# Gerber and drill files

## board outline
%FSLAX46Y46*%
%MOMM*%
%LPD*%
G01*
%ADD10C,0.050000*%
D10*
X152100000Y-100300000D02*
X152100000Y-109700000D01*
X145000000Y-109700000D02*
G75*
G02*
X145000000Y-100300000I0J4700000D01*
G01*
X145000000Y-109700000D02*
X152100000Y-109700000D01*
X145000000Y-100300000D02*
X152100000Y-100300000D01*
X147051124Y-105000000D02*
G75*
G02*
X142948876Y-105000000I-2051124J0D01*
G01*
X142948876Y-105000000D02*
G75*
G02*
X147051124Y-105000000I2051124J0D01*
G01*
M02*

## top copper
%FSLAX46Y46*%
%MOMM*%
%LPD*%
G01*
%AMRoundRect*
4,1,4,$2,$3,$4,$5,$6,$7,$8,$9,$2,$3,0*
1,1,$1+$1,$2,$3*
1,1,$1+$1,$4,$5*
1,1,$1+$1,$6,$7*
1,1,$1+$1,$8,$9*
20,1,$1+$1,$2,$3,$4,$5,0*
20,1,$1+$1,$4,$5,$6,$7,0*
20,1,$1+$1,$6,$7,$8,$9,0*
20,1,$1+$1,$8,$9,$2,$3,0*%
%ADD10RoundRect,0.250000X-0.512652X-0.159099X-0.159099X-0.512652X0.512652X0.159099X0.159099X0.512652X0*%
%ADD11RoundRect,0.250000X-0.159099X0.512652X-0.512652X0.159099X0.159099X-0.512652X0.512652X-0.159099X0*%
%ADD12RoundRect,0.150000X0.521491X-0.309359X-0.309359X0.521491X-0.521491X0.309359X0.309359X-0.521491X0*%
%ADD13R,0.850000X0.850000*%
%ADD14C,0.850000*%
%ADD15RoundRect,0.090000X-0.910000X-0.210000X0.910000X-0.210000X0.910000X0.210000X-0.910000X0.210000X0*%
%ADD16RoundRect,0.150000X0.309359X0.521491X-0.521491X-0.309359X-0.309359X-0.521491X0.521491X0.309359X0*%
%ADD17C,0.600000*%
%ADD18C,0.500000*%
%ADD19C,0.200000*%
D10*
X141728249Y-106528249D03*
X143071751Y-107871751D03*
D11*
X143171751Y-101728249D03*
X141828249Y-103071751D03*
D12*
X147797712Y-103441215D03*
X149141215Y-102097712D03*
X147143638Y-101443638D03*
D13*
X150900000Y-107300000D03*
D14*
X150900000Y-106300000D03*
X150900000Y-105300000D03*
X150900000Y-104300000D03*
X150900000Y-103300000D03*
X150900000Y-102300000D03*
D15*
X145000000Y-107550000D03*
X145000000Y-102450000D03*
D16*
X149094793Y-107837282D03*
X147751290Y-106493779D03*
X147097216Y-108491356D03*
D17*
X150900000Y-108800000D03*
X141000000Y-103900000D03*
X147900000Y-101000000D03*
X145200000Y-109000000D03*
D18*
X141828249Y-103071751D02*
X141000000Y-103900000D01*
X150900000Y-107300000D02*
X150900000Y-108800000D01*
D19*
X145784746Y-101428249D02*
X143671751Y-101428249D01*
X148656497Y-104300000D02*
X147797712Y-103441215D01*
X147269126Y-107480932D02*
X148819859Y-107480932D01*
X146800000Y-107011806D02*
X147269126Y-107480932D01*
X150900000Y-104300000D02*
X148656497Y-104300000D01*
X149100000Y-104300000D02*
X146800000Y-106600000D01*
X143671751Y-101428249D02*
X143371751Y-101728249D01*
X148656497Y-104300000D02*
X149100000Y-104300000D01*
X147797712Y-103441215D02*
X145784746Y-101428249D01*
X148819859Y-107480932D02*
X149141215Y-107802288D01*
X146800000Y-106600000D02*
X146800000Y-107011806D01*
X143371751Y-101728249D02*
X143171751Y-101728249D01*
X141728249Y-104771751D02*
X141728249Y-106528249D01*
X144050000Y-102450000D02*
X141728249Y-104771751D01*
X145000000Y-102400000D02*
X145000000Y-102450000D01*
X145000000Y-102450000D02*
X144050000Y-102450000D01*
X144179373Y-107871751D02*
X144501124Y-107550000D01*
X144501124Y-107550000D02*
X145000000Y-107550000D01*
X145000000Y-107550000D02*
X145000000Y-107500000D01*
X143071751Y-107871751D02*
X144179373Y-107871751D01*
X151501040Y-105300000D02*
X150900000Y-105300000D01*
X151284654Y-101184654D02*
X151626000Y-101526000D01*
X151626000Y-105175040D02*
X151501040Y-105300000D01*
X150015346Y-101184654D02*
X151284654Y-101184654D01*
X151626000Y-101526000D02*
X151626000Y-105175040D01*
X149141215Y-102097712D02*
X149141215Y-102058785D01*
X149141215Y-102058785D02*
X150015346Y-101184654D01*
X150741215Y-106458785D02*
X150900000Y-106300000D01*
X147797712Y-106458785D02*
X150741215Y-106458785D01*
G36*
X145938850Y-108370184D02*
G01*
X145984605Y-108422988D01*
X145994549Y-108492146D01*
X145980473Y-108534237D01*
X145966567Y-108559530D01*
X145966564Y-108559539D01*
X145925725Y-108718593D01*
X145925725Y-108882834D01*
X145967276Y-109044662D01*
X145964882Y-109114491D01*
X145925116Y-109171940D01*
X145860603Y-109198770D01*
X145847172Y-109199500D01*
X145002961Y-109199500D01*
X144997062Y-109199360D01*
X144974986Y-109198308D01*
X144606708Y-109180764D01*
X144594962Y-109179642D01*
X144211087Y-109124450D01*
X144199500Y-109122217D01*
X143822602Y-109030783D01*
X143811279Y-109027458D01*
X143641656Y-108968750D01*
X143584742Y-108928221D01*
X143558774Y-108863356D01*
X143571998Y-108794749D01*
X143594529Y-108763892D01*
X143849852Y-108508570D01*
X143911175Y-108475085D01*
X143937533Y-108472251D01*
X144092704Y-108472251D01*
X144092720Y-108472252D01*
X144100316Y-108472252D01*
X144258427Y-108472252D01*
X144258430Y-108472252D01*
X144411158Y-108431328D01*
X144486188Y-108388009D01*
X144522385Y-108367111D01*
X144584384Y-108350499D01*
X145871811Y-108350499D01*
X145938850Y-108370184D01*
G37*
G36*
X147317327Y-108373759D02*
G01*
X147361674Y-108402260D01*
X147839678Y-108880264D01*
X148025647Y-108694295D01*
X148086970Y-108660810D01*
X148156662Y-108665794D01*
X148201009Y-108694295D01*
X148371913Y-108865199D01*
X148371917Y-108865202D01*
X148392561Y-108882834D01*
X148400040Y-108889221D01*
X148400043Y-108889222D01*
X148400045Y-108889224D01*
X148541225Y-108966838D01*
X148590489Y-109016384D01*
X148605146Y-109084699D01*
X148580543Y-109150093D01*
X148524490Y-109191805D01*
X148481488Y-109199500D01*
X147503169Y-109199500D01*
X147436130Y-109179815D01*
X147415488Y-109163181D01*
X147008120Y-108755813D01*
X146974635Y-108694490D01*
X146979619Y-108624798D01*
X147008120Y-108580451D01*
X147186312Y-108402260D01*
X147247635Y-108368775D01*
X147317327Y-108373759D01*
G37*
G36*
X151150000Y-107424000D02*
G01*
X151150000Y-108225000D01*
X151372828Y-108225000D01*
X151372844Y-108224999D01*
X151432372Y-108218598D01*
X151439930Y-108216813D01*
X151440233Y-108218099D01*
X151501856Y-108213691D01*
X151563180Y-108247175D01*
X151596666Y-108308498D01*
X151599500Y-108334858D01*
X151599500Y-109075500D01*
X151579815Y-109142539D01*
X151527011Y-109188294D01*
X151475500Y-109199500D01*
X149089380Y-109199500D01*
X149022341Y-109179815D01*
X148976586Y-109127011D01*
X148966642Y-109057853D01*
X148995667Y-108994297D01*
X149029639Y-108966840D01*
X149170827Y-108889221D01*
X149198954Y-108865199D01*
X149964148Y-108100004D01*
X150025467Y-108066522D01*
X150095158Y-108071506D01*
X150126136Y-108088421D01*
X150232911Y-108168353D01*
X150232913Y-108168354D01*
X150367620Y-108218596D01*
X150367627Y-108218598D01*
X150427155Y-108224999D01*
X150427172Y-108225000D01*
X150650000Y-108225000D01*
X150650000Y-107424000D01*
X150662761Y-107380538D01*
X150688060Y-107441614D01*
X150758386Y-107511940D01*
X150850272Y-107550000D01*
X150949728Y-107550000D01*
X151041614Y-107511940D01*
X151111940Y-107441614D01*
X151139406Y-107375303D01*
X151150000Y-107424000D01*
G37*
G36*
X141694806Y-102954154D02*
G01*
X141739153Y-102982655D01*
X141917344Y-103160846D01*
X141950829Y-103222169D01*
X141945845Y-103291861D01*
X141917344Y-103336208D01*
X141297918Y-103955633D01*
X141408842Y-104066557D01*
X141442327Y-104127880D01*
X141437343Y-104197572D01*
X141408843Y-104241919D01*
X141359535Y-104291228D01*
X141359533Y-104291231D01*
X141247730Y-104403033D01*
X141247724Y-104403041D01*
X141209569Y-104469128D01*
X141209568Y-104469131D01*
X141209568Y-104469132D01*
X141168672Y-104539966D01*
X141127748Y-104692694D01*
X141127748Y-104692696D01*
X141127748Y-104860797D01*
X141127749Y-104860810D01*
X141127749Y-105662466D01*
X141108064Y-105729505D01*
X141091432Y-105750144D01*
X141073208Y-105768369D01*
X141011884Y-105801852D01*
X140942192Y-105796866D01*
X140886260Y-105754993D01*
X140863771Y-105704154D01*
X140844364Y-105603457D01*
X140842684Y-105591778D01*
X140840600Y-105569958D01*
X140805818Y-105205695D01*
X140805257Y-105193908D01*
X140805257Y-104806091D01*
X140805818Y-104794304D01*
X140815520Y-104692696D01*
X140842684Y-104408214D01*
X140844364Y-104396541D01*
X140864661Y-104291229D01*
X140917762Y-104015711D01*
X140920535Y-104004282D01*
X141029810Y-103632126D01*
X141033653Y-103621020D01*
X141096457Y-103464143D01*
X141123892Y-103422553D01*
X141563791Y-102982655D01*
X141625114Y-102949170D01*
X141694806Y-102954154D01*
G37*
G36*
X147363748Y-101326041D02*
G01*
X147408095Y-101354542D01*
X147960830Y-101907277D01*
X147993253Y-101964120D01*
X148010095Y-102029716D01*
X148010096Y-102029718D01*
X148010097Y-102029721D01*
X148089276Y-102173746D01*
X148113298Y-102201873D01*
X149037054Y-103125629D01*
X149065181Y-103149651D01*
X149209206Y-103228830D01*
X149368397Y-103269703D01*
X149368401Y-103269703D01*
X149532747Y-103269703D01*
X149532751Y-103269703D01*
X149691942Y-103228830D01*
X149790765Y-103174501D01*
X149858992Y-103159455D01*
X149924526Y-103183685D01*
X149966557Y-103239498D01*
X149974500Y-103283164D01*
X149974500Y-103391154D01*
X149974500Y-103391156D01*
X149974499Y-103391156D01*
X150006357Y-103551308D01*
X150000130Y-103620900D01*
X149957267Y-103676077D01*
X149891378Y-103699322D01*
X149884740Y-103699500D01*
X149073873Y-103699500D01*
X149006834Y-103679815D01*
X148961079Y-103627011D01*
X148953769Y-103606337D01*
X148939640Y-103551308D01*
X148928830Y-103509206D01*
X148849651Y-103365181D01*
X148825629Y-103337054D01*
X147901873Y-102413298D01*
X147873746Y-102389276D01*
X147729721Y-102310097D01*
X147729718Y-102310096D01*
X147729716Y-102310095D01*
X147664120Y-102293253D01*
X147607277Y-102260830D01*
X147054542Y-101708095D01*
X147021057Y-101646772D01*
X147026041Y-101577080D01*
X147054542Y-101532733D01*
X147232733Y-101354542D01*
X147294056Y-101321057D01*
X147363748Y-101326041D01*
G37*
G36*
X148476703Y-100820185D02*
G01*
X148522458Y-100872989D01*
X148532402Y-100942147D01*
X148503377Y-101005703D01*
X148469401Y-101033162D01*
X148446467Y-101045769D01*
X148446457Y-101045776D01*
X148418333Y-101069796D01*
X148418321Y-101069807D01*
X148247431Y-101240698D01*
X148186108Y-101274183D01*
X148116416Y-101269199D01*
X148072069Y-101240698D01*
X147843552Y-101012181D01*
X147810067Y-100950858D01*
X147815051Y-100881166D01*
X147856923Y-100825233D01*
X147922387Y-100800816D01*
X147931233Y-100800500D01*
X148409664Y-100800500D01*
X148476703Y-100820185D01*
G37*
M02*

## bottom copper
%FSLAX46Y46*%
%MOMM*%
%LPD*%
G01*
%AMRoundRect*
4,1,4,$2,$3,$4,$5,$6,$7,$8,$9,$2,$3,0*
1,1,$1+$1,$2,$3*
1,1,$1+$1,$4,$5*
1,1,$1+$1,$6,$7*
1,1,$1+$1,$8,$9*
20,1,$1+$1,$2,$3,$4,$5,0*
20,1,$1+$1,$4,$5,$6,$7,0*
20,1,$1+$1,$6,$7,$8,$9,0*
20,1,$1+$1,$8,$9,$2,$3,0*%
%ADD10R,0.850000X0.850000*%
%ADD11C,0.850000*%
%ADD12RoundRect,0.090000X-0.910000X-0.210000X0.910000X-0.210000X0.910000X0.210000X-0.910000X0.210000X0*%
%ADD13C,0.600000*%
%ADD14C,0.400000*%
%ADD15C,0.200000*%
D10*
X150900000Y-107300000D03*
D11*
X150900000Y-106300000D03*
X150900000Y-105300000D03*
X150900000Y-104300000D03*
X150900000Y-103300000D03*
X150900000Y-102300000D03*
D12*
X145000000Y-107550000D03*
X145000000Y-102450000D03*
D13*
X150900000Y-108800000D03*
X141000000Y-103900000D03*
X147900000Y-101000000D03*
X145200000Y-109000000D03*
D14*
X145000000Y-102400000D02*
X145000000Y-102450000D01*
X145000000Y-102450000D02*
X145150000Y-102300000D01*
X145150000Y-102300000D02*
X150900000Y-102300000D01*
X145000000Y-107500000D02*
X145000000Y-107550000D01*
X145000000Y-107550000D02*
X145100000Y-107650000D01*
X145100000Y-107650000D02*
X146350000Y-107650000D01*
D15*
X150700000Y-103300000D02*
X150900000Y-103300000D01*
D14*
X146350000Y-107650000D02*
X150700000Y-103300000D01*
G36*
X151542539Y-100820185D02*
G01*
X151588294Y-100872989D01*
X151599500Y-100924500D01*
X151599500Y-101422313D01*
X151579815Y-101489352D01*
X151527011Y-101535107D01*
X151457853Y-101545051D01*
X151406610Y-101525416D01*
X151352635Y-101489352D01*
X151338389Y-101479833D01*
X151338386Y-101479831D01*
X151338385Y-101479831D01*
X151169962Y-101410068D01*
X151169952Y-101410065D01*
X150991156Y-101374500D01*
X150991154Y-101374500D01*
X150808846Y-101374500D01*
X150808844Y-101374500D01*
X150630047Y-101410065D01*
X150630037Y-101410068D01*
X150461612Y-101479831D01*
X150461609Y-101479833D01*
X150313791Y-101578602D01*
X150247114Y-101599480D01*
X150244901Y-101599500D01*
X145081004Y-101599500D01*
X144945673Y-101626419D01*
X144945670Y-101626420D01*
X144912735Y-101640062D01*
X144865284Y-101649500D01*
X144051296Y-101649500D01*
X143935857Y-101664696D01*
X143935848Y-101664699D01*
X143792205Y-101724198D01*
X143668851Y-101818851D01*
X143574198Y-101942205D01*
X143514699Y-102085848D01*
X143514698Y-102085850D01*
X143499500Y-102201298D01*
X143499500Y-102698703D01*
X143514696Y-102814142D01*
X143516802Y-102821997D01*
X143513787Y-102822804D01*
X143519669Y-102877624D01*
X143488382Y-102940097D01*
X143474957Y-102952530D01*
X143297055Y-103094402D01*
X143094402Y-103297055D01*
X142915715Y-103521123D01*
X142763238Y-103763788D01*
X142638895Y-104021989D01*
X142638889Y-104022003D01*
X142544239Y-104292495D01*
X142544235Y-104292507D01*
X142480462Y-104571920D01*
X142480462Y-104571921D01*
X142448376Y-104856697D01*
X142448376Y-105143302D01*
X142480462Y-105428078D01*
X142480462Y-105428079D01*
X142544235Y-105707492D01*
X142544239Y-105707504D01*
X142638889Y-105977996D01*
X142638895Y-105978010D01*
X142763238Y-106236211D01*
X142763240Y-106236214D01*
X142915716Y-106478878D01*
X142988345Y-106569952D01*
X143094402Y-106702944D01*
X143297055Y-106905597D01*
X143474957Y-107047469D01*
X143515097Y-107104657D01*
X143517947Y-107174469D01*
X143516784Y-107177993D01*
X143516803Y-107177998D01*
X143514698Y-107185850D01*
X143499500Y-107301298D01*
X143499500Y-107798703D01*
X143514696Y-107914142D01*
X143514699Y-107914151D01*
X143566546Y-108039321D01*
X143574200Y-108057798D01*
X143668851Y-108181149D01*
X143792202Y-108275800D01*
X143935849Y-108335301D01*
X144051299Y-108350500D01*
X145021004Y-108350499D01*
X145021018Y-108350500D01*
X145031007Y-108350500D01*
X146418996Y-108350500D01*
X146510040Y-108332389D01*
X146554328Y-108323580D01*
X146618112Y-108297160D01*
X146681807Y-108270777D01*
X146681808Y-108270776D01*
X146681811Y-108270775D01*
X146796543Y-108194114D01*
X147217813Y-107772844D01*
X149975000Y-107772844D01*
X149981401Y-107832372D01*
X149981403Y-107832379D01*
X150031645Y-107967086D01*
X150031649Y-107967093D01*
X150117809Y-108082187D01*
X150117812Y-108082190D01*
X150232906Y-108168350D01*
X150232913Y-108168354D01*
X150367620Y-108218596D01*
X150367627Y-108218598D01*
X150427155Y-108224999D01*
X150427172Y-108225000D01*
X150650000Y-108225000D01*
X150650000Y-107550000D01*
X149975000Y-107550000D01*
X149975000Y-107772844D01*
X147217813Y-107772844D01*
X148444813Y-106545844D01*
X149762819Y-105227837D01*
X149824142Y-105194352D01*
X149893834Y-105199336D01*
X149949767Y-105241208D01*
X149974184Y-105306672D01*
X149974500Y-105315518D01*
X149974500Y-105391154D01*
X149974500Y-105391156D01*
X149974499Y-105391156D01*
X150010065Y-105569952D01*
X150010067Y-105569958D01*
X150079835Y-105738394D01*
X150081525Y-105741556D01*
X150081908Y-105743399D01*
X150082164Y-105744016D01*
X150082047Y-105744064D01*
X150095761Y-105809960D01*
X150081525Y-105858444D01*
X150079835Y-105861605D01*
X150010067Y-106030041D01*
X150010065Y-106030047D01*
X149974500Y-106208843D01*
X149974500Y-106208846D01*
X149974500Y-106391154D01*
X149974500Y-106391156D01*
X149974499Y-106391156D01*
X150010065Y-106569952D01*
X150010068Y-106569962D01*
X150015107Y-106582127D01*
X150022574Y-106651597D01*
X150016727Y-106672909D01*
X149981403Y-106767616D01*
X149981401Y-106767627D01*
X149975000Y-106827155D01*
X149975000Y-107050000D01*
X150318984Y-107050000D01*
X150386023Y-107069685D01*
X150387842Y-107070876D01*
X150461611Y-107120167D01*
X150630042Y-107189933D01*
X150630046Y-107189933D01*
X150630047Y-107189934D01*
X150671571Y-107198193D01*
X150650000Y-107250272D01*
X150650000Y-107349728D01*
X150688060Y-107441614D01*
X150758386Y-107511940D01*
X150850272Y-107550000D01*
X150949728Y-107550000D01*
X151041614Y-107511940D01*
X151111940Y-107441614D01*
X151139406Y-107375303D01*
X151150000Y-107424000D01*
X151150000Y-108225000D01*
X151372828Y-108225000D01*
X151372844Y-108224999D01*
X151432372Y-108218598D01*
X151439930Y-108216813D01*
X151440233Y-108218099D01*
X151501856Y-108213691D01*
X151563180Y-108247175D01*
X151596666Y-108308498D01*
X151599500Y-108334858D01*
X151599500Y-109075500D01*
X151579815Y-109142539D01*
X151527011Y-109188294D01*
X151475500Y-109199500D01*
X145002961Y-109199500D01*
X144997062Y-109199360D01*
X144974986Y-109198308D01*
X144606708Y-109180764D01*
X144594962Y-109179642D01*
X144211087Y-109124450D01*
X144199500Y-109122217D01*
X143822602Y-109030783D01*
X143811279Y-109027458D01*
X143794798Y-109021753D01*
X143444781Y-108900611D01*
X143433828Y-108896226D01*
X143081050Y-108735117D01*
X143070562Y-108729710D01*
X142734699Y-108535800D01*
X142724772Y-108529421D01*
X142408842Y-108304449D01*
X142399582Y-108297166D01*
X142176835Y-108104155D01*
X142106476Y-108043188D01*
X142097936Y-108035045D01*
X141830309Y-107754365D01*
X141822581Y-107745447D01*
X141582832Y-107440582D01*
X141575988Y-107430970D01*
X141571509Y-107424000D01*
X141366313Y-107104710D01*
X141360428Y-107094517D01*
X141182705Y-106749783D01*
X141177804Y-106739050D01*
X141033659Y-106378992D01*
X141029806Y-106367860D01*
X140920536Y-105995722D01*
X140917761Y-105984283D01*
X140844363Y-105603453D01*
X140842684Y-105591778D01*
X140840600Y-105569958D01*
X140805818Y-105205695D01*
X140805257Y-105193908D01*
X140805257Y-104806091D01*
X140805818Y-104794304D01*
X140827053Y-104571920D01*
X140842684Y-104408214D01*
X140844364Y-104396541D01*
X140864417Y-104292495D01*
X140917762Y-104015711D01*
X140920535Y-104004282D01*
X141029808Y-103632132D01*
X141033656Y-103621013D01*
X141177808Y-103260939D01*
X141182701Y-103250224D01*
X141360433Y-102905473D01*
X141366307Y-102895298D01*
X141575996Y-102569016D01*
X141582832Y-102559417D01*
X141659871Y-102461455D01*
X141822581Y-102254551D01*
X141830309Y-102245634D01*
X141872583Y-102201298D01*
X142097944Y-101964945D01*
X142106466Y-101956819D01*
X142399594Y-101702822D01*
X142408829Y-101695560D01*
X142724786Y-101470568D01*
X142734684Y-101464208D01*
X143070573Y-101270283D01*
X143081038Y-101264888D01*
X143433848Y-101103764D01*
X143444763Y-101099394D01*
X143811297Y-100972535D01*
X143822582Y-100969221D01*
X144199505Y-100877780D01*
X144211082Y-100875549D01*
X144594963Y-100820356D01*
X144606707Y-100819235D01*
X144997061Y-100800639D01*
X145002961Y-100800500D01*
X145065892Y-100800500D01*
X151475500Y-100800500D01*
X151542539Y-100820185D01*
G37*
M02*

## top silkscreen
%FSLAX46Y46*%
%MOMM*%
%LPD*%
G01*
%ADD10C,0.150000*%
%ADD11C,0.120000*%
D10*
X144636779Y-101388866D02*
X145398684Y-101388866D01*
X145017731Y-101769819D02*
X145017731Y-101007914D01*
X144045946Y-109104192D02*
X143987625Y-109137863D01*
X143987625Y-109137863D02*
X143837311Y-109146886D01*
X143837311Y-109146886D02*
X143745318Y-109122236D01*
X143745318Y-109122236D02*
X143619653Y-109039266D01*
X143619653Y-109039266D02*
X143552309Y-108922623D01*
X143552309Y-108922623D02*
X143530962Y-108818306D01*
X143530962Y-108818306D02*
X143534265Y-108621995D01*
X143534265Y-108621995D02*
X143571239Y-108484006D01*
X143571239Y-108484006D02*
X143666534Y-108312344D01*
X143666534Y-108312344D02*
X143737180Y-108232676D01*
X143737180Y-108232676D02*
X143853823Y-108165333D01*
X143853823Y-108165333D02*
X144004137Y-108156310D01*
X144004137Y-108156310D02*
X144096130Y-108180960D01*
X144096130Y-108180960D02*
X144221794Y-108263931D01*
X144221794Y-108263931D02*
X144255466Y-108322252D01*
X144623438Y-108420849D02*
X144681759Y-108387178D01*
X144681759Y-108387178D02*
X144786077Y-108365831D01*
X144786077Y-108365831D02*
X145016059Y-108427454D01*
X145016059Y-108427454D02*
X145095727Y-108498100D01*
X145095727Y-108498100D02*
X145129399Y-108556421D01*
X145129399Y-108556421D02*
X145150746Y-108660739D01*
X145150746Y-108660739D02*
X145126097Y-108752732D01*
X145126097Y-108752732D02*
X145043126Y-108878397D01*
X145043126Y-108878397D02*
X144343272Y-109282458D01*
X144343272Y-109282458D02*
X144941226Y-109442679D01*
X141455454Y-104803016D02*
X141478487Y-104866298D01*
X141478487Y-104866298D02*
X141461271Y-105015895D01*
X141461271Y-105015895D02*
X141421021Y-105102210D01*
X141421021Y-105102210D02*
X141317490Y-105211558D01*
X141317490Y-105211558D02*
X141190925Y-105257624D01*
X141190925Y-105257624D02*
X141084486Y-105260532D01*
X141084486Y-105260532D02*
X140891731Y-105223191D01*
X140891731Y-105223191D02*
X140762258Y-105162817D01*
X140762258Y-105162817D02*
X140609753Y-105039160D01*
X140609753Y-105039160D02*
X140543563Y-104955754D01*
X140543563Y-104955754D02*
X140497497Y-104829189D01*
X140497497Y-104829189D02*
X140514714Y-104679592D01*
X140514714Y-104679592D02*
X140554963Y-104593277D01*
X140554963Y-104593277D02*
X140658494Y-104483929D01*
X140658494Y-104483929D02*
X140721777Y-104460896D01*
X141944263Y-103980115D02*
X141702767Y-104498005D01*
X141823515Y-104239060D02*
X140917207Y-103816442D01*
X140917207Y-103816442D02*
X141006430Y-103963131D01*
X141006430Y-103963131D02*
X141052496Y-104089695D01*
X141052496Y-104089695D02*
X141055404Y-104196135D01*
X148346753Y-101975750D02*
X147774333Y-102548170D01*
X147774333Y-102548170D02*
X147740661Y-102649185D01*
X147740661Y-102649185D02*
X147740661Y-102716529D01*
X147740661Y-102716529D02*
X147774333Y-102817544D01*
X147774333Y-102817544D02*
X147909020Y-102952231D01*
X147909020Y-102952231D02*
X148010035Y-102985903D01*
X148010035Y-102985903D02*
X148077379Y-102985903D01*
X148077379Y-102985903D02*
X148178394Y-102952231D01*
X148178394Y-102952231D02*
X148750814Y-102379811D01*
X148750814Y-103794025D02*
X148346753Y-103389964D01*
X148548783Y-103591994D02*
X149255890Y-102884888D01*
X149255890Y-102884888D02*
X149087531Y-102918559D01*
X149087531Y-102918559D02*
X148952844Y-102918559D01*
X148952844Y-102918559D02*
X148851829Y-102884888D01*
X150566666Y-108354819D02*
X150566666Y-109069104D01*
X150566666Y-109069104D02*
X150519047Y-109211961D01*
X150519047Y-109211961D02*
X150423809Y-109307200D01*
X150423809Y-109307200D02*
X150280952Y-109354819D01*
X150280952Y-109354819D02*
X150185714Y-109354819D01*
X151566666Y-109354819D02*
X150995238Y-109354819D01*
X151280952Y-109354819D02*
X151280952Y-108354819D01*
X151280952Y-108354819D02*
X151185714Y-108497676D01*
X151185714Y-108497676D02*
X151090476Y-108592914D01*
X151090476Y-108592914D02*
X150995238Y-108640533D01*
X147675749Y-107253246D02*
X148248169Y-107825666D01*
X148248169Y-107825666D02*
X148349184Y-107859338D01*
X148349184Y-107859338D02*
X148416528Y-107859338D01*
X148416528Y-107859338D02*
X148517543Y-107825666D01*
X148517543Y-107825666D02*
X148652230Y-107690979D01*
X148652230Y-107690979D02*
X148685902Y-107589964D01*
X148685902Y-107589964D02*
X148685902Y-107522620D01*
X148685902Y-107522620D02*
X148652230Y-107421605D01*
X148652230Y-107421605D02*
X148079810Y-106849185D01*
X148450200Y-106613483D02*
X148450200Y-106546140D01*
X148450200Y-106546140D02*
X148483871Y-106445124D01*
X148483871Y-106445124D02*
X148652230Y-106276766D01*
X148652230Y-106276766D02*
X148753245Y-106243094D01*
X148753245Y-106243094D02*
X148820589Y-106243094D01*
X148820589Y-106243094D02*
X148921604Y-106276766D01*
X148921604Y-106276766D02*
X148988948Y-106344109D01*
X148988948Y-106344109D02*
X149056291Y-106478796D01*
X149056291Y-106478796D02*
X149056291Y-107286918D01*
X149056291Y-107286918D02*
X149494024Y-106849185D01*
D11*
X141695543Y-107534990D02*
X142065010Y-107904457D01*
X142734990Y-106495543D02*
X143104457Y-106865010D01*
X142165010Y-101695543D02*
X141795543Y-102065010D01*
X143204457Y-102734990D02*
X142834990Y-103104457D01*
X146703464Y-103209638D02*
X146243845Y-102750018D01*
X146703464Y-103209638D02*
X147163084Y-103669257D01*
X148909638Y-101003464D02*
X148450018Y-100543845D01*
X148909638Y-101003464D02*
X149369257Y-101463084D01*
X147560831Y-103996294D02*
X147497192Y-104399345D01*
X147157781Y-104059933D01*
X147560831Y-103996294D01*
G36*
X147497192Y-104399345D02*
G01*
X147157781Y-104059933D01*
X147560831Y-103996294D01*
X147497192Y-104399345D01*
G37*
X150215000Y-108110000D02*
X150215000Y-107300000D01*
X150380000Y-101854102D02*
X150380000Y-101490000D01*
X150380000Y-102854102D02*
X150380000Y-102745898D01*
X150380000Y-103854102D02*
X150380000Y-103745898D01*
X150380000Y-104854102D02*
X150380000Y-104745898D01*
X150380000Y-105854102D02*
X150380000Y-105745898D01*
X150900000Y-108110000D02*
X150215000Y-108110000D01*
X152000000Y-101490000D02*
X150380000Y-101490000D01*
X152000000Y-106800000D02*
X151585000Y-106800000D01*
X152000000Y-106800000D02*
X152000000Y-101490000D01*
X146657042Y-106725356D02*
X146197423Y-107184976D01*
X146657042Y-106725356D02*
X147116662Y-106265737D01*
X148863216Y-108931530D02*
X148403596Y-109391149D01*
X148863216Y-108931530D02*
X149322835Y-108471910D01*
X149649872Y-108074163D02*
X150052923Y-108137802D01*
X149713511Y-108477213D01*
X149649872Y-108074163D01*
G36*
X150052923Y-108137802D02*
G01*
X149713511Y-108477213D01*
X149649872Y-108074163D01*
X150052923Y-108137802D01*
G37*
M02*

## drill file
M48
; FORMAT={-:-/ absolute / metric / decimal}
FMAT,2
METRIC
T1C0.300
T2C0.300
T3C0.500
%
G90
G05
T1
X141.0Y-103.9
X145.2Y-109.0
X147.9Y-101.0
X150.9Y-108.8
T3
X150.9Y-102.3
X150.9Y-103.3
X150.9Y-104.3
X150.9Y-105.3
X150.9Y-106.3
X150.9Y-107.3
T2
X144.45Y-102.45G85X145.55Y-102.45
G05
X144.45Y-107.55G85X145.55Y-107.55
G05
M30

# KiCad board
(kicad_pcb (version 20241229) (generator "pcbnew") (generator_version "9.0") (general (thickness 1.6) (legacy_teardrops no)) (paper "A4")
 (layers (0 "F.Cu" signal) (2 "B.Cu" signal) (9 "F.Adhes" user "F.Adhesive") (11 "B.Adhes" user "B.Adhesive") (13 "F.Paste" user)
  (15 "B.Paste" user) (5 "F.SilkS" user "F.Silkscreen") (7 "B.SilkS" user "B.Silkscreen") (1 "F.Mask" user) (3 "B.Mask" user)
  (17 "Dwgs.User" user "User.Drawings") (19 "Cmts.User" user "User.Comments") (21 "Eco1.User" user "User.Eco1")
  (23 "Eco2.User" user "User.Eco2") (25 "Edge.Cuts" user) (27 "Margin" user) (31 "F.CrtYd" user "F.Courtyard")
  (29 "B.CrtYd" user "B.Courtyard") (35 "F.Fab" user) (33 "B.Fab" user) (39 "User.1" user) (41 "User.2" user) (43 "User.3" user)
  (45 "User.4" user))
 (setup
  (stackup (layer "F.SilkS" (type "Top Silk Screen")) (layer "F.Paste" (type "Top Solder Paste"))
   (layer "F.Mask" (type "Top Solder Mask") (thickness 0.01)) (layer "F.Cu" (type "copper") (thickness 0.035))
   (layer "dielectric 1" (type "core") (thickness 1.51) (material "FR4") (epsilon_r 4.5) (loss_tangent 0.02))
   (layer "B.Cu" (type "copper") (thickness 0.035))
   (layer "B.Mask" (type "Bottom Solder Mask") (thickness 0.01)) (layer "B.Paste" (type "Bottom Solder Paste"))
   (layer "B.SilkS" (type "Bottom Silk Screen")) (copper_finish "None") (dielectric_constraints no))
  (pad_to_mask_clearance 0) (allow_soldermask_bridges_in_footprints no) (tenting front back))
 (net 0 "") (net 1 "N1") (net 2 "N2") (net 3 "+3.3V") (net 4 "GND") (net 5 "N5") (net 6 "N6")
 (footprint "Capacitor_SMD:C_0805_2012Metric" (layer "F.Cu") (at 142.4 107.2 -45)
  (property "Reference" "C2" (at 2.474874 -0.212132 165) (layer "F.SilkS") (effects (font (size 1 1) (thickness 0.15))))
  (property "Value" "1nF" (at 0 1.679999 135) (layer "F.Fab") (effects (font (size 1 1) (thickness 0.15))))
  (fp_line (start -0.261253 0.735) (end 0.261253 0.735) (stroke (width 0.12) (type solid)) (layer "F.SilkS"))
  (fp_line (start -0.261253 -0.735) (end 0.261253 -0.735) (stroke (width 0.12) (type solid)) (layer "F.SilkS"))
  (pad "1" smd roundrect (at -0.949999 0 315) (size 1 1.45) (layers "F.Cu" "F.Mask" "F.Paste") (roundrect_rratio 0.25) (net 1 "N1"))
  (pad "2" smd roundrect (at 0.949999 0 315) (size 1 1.45) (layers "F.Cu" "F.Mask" "F.Paste") (roundrect_rratio 0.25) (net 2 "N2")))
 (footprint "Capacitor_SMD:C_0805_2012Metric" (layer "F.Cu") (at 142.5 102.4 -135)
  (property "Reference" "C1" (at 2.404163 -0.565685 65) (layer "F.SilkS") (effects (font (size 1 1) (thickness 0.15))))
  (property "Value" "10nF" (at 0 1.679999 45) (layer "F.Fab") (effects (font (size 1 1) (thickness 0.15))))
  (fp_line (start -0.261253 0.735) (end 0.261253 0.735) (stroke (width 0.12) (type solid)) (layer "F.SilkS"))
  (fp_line (start -0.261253 -0.735) (end 0.261253 -0.735) (stroke (width 0.12) (type solid)) (layer "F.SilkS"))
  (pad "1" smd roundrect (at -0.949999 0 225) (size 1 1.45) (layers "F.Cu" "F.Mask" "F.Paste") (roundrect_rratio 0.25) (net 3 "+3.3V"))
  (pad "2" smd roundrect (at 0.949999 0 225) (size 1 1.45) (layers "F.Cu" "F.Mask" "F.Paste") (roundrect_rratio 0.25) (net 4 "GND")))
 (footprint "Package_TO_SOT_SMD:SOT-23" (layer "F.Cu") (at 147.806551 102.106551 135)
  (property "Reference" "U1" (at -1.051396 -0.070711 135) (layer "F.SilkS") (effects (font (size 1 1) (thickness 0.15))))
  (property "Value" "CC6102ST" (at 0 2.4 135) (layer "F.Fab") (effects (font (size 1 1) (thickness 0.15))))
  (fp_line (start 0 -1.560001) (end 0.65 -1.56) (stroke (width 0.12) (type solid)) (layer "F.SilkS"))
  (fp_line (start 0 -1.560001) (end -0.65 -1.56) (stroke (width 0.12) (type solid)) (layer "F.SilkS"))
  (fp_line (start 0 1.560001) (end 0.65 1.56) (stroke (width 0.12) (type solid)) (layer "F.SilkS"))
  (fp_line (start 0 1.560001) (end -0.65 1.56) (stroke (width 0.12) (type solid)) (layer "F.SilkS"))
  (fp_poly
   (pts (xy -1.1625 -1.51) (xy -1.4025 -1.84) (xy -0.9225 -1.839999)) (stroke (width 0.12) (type solid)) (fill yes) (layer "F.SilkS"))
  (pad "1" smd roundrect (at -0.9375 -0.95 135) (size 1.475 0.6) (layers "F.Cu" "F.Mask" "F.Paste") (roundrect_rratio 0.25) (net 3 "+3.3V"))
  (pad "2" smd roundrect (at -0.9375 0.95 135) (size 1.475 0.6) (layers "F.Cu" "F.Mask" "F.Paste") (roundrect_rratio 0.25) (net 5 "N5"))
  (pad "3" smd roundrect (at 0.937501 0 135) (size 1.475 0.6) (layers "F.Cu" "F.Mask" "F.Paste") (roundrect_rratio 0.25) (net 4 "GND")))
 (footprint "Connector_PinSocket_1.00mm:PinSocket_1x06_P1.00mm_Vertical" (layer "F.Cu") (at 150.9 107.3 180)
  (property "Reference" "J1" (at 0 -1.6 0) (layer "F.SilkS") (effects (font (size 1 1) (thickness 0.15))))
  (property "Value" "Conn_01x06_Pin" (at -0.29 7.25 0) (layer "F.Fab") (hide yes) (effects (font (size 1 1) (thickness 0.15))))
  (fp_line (start 0.685 -0.81) (end 0.685 0) (stroke (width 0.12) (type solid)) (layer "F.SilkS"))
  (fp_line (start 0.52 5.445898) (end 0.52 5.81) (stroke (width 0.12) (type solid)) (layer "F.SilkS"))
  (fp_line (start 0.52 4.445898) (end 0.52 4.554102) (stroke (width 0.12) (type solid)) (layer "F.SilkS"))
  (fp_line (start 0.52 3.445898) (end 0.52 3.554102) (stroke (width 0.12) (type solid)) (layer "F.SilkS"))
  (fp_line (start 0.52 2.445898) (end 0.52 2.554102) (stroke (width 0.12) (type solid)) (layer "F.SilkS"))
  (fp_line (start 0.52 1.445898) (end 0.52 1.554102) (stroke (width 0.12) (type solid)) (layer "F.SilkS"))
  (fp_line (start 0 -0.81) (end 0.685 -0.81) (stroke (width 0.12) (type solid)) (layer "F.SilkS"))
  (fp_line (start -1.1 5.81) (end 0.52 5.81) (stroke (width 0.12) (type solid)) (layer "F.SilkS"))
  (fp_line (start -1.1 0.5) (end -0.685 0.5) (stroke (width 0.12) (type solid)) (layer "F.SilkS"))
  (fp_line (start -1.1 0.5) (end -1.1 5.81) (stroke (width 0.12) (type solid)) (layer "F.SilkS"))
  (pad "1" thru_hole rect (at 0 0 180) (size 0.85 0.85) (drill 0.5) (layers "*.Cu" "*.Mask") (remove_unused_layers no) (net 4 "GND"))
  (pad "2" thru_hole circle (at 0 1 180) (size 0.85 0.85) (drill 0.5) (layers "*.Cu" "*.Mask") (remove_unused_layers no) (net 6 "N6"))
  (pad "3" thru_hole circle (at 0 2 180) (size 0.85 0.85) (drill 0.5) (layers "*.Cu" "*.Mask") (remove_unused_layers no) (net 5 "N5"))
  (pad "4" thru_hole circle (at 0 3 180) (size 0.85 0.85) (drill 0.5) (layers "*.Cu" "*.Mask") (remove_unused_layers no) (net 3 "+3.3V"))
  (pad "5" thru_hole circle (at 0 4 180) (size 0.85 0.85) (drill 0.5) (layers "*.Cu" "*.Mask") (remove_unused_layers no) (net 2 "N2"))
  (pad "6" thru_hole circle (at 0 5 180) (size 0.85 0.85) (drill 0.5) (layers "*.Cu" "*.Mask") (remove_unused_layers no) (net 1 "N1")))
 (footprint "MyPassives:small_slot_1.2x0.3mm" (layer "F.Cu") (at 145 109.836)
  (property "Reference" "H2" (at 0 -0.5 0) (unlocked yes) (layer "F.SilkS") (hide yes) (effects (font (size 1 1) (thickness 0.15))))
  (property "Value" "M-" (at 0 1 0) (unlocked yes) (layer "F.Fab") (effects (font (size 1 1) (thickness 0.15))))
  (pad "1" thru_hole roundrect (at 0 -2.286) (size 2 0.6) (drill oval 1.4 0.3) (layers "*.Cu" "*.Mask") (remove_unused_layers no)
   (roundrect_rratio 0.15) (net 2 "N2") (thermal_bridge_angle 45)))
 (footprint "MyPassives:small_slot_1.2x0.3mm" (layer "F.Cu") (at 145 104.736)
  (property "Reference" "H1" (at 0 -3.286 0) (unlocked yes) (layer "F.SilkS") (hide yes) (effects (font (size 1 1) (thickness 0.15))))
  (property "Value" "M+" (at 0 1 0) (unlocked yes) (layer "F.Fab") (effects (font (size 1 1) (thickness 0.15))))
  (pad "1" thru_hole roundrect (at 0 -2.286) (size 2 0.6) (drill oval 1.4 0.3) (layers "*.Cu" "*.Mask") (remove_unused_layers no)
   (roundrect_rratio 0.15) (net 1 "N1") (thermal_bridge_angle 45)))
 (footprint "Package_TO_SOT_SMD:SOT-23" (layer "F.Cu") (at 147.760129 107.828443 -135)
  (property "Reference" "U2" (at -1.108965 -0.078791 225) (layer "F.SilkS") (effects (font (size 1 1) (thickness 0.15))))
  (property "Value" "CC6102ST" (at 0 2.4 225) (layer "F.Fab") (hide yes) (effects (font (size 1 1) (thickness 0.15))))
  (fp_line (start 0 1.560001) (end 0.65 1.56) (stroke (width 0.12) (type solid)) (layer "F.SilkS"))
  (fp_line (start 0 1.560001) (end -0.65 1.56) (stroke (width 0.12) (type solid)) (layer "F.SilkS"))
  (fp_line (start 0 -1.560001) (end 0.65 -1.56) (stroke (width 0.12) (type solid)) (layer "F.SilkS"))
  (fp_line (start 0 -1.560001) (end -0.65 -1.56) (stroke (width 0.12) (type solid)) (layer "F.SilkS"))
  (fp_poly
   (pts (xy -1.1625 -1.51) (xy -1.4025 -1.84) (xy -0.9225 -1.839999)) (stroke (width 0.12) (type solid)) (fill yes) (layer "F.SilkS"))
  (pad "1" smd roundrect (at -0.9375 -0.95 225) (size 1.475 0.6) (layers "F.Cu" "F.Mask" "F.Paste") (roundrect_rratio 0.25) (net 3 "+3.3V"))
  (pad "2" smd roundrect (at -0.9375 0.95 225) (size 1.475 0.6) (layers "F.Cu" "F.Mask" "F.Paste") (roundrect_rratio 0.25) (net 6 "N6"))
  (pad "3" smd roundrect (at 0.937501 0 225) (size 1.475 0.6) (layers "F.Cu" "F.Mask" "F.Paste") (roundrect_rratio 0.25) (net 4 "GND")))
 (gr_line (start 152.1 100.3) (end 152.1 109.7) (stroke (width 0.05) (type default)) (locked yes) (layer "Edge.Cuts"))
 (gr_arc (start 145 109.7) (mid 140.3 105) (end 145 100.3) (stroke (width 0.05) (type default)) (locked yes) (layer "Edge.Cuts"))
 (gr_line (start 145 109.7) (end 152.1 109.7) (stroke (width 0.05) (type default)) (locked yes) (layer "Edge.Cuts"))
 (gr_line (start 145 100.3) (end 152.1 100.3) (stroke (width 0.05) (type default)) (locked yes) (layer "Edge.Cuts"))
 (gr_circle (center 145 105) (end 144.975034 107.050972) (stroke (width 0.05) (type default)) (fill no) (layer "Edge.Cuts"))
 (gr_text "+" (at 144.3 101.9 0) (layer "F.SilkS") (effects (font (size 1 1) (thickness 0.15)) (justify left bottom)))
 (segment (start 141.828249 103.071751) (end 141 103.9) (width 0.5) (layer "F.Cu") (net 4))
 (segment (start 150.9 107.3) (end 150.9 108.8) (width 0.5) (layer "F.Cu") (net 4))
 (via (at 150.9 108.8) (size 0.6) (drill 0.3) (layers "F.Cu" "B.Cu") (free yes) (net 4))
 (via (at 141 103.9) (size 0.6) (drill 0.3) (layers "F.Cu" "B.Cu") (free yes) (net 4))
 (via (at 147.9 101) (size 0.6) (drill 0.3) (layers "F.Cu" "B.Cu") (free yes) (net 4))
 (via (at 145.2 109) (size 0.6) (drill 0.3) (layers "F.Cu" "B.Cu") (free yes) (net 4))
 (segment (start 145.784746 101.428249) (end 143.671751 101.428249) (width 0.2) (layer "F.Cu") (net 3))
 (segment (start 148.656497 104.3) (end 147.797712 103.441215) (width 0.2) (layer "F.Cu") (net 3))
 (segment (start 147.269126 107.480932) (end 148.819859 107.480932) (width 0.2) (layer "F.Cu") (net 3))
 (segment (start 146.8 107.011806) (end 147.269126 107.480932) (width 0.2) (layer "F.Cu") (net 3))
 (segment (start 150.9 104.3) (end 148.656497 104.3) (width 0.2) (layer "F.Cu") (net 3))
 (segment (start 149.1 104.3) (end 146.8 106.6) (width 0.2) (layer "F.Cu") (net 3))
 (segment (start 143.671751 101.428249) (end 143.371751 101.728249) (width 0.2) (layer "F.Cu") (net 3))
 (segment (start 148.656497 104.3) (end 149.1 104.3) (width 0.2) (layer "F.Cu") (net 3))
 (segment (start 147.797712 103.441215) (end 145.784746 101.428249) (width 0.2) (layer "F.Cu") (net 3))
 (segment (start 148.819859 107.480932) (end 149.141215 107.802288) (width 0.2) (layer "F.Cu") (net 3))
 (segment (start 146.8 106.6) (end 146.8 107.011806) (width 0.2) (layer "F.Cu") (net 3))
 (segment (start 143.371751 101.728249) (end 143.171751 101.728249) (width 0.2) (layer "F.Cu") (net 3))
 (segment (start 141.728249 104.771751) (end 141.728249 106.528249) (width 0.2) (layer "F.Cu") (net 1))
 (segment (start 144.05 102.45) (end 141.728249 104.771751) (width 0.2) (layer "F.Cu") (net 1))
 (segment (start 145 102.4) (end 145 102.45) (width 0.2) (layer "F.Cu") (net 1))
 (segment (start 145 102.45) (end 144.05 102.45) (width 0.2) (layer "F.Cu") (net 1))
 (segment (start 145 102.4) (end 145 102.45) (width 0.4) (layer "B.Cu") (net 1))
 (segment (start 145 102.45) (end 145.15 102.3) (width 0.4) (layer "B.Cu") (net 1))
 (segment (start 145.15 102.3) (end 150.9 102.3) (width 0.4) (layer "B.Cu") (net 1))
 (segment (start 144.179373 107.871751) (end 144.501124 107.55) (width 0.2) (layer "F.Cu") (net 2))
 (segment (start 144.501124 107.55) (end 145 107.55) (width 0.2) (layer "F.Cu") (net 2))
 (segment (start 145 107.55) (end 145 107.5) (width 0.2) (layer "F.Cu") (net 2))
 (segment (start 143.071751 107.871751) (end 144.179373 107.871751) (width 0.2) (layer "F.Cu") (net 2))
 (segment (start 145 107.5) (end 145 107.55) (width 0.4) (layer "B.Cu") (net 2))
 (segment (start 145 107.55) (end 145.1 107.65) (width 0.4) (layer "B.Cu") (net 2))
 (segment (start 145.1 107.65) (end 146.35 107.65) (width 0.4) (layer "B.Cu") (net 2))
 (segment (start 150.7 103.3) (end 150.9 103.3) (width 0.2) (layer "B.Cu") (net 2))
 (segment (start 146.35 107.65) (end 150.7 103.3) (width 0.4) (layer "B.Cu") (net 2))
 (segment (start 151.50104 105.3) (end 150.9 105.3) (width 0.2) (layer "F.Cu") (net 5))
 (segment (start 151.284654 101.184654) (end 151.626 101.526) (width 0.2) (layer "F.Cu") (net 5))
 (segment (start 151.626 105.17504) (end 151.50104 105.3) (width 0.2) (layer "F.Cu") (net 5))
 (segment (start 150.015346 101.184654) (end 151.284654 101.184654) (width 0.2) (layer "F.Cu") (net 5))
 (segment (start 151.626 101.526) (end 151.626 105.17504) (width 0.2) (layer "F.Cu") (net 5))
 (segment (start 149.141215 102.097712) (end 149.141215 102.058785) (width 0.2) (layer "F.Cu") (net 5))
 (segment (start 149.141215 102.058785) (end 150.015346 101.184654) (width 0.2) (layer "F.Cu") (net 5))
 (segment (start 150.741215 106.458785) (end 150.9 106.3) (width 0.2) (layer "F.Cu") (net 6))
 (segment (start 147.797712 106.458785) (end 150.741215 106.458785) (width 0.2) (layer "F.Cu") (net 6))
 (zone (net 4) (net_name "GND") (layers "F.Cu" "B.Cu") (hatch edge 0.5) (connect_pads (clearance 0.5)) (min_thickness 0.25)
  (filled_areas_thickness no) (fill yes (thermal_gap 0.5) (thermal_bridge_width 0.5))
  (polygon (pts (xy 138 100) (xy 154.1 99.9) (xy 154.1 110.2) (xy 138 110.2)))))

